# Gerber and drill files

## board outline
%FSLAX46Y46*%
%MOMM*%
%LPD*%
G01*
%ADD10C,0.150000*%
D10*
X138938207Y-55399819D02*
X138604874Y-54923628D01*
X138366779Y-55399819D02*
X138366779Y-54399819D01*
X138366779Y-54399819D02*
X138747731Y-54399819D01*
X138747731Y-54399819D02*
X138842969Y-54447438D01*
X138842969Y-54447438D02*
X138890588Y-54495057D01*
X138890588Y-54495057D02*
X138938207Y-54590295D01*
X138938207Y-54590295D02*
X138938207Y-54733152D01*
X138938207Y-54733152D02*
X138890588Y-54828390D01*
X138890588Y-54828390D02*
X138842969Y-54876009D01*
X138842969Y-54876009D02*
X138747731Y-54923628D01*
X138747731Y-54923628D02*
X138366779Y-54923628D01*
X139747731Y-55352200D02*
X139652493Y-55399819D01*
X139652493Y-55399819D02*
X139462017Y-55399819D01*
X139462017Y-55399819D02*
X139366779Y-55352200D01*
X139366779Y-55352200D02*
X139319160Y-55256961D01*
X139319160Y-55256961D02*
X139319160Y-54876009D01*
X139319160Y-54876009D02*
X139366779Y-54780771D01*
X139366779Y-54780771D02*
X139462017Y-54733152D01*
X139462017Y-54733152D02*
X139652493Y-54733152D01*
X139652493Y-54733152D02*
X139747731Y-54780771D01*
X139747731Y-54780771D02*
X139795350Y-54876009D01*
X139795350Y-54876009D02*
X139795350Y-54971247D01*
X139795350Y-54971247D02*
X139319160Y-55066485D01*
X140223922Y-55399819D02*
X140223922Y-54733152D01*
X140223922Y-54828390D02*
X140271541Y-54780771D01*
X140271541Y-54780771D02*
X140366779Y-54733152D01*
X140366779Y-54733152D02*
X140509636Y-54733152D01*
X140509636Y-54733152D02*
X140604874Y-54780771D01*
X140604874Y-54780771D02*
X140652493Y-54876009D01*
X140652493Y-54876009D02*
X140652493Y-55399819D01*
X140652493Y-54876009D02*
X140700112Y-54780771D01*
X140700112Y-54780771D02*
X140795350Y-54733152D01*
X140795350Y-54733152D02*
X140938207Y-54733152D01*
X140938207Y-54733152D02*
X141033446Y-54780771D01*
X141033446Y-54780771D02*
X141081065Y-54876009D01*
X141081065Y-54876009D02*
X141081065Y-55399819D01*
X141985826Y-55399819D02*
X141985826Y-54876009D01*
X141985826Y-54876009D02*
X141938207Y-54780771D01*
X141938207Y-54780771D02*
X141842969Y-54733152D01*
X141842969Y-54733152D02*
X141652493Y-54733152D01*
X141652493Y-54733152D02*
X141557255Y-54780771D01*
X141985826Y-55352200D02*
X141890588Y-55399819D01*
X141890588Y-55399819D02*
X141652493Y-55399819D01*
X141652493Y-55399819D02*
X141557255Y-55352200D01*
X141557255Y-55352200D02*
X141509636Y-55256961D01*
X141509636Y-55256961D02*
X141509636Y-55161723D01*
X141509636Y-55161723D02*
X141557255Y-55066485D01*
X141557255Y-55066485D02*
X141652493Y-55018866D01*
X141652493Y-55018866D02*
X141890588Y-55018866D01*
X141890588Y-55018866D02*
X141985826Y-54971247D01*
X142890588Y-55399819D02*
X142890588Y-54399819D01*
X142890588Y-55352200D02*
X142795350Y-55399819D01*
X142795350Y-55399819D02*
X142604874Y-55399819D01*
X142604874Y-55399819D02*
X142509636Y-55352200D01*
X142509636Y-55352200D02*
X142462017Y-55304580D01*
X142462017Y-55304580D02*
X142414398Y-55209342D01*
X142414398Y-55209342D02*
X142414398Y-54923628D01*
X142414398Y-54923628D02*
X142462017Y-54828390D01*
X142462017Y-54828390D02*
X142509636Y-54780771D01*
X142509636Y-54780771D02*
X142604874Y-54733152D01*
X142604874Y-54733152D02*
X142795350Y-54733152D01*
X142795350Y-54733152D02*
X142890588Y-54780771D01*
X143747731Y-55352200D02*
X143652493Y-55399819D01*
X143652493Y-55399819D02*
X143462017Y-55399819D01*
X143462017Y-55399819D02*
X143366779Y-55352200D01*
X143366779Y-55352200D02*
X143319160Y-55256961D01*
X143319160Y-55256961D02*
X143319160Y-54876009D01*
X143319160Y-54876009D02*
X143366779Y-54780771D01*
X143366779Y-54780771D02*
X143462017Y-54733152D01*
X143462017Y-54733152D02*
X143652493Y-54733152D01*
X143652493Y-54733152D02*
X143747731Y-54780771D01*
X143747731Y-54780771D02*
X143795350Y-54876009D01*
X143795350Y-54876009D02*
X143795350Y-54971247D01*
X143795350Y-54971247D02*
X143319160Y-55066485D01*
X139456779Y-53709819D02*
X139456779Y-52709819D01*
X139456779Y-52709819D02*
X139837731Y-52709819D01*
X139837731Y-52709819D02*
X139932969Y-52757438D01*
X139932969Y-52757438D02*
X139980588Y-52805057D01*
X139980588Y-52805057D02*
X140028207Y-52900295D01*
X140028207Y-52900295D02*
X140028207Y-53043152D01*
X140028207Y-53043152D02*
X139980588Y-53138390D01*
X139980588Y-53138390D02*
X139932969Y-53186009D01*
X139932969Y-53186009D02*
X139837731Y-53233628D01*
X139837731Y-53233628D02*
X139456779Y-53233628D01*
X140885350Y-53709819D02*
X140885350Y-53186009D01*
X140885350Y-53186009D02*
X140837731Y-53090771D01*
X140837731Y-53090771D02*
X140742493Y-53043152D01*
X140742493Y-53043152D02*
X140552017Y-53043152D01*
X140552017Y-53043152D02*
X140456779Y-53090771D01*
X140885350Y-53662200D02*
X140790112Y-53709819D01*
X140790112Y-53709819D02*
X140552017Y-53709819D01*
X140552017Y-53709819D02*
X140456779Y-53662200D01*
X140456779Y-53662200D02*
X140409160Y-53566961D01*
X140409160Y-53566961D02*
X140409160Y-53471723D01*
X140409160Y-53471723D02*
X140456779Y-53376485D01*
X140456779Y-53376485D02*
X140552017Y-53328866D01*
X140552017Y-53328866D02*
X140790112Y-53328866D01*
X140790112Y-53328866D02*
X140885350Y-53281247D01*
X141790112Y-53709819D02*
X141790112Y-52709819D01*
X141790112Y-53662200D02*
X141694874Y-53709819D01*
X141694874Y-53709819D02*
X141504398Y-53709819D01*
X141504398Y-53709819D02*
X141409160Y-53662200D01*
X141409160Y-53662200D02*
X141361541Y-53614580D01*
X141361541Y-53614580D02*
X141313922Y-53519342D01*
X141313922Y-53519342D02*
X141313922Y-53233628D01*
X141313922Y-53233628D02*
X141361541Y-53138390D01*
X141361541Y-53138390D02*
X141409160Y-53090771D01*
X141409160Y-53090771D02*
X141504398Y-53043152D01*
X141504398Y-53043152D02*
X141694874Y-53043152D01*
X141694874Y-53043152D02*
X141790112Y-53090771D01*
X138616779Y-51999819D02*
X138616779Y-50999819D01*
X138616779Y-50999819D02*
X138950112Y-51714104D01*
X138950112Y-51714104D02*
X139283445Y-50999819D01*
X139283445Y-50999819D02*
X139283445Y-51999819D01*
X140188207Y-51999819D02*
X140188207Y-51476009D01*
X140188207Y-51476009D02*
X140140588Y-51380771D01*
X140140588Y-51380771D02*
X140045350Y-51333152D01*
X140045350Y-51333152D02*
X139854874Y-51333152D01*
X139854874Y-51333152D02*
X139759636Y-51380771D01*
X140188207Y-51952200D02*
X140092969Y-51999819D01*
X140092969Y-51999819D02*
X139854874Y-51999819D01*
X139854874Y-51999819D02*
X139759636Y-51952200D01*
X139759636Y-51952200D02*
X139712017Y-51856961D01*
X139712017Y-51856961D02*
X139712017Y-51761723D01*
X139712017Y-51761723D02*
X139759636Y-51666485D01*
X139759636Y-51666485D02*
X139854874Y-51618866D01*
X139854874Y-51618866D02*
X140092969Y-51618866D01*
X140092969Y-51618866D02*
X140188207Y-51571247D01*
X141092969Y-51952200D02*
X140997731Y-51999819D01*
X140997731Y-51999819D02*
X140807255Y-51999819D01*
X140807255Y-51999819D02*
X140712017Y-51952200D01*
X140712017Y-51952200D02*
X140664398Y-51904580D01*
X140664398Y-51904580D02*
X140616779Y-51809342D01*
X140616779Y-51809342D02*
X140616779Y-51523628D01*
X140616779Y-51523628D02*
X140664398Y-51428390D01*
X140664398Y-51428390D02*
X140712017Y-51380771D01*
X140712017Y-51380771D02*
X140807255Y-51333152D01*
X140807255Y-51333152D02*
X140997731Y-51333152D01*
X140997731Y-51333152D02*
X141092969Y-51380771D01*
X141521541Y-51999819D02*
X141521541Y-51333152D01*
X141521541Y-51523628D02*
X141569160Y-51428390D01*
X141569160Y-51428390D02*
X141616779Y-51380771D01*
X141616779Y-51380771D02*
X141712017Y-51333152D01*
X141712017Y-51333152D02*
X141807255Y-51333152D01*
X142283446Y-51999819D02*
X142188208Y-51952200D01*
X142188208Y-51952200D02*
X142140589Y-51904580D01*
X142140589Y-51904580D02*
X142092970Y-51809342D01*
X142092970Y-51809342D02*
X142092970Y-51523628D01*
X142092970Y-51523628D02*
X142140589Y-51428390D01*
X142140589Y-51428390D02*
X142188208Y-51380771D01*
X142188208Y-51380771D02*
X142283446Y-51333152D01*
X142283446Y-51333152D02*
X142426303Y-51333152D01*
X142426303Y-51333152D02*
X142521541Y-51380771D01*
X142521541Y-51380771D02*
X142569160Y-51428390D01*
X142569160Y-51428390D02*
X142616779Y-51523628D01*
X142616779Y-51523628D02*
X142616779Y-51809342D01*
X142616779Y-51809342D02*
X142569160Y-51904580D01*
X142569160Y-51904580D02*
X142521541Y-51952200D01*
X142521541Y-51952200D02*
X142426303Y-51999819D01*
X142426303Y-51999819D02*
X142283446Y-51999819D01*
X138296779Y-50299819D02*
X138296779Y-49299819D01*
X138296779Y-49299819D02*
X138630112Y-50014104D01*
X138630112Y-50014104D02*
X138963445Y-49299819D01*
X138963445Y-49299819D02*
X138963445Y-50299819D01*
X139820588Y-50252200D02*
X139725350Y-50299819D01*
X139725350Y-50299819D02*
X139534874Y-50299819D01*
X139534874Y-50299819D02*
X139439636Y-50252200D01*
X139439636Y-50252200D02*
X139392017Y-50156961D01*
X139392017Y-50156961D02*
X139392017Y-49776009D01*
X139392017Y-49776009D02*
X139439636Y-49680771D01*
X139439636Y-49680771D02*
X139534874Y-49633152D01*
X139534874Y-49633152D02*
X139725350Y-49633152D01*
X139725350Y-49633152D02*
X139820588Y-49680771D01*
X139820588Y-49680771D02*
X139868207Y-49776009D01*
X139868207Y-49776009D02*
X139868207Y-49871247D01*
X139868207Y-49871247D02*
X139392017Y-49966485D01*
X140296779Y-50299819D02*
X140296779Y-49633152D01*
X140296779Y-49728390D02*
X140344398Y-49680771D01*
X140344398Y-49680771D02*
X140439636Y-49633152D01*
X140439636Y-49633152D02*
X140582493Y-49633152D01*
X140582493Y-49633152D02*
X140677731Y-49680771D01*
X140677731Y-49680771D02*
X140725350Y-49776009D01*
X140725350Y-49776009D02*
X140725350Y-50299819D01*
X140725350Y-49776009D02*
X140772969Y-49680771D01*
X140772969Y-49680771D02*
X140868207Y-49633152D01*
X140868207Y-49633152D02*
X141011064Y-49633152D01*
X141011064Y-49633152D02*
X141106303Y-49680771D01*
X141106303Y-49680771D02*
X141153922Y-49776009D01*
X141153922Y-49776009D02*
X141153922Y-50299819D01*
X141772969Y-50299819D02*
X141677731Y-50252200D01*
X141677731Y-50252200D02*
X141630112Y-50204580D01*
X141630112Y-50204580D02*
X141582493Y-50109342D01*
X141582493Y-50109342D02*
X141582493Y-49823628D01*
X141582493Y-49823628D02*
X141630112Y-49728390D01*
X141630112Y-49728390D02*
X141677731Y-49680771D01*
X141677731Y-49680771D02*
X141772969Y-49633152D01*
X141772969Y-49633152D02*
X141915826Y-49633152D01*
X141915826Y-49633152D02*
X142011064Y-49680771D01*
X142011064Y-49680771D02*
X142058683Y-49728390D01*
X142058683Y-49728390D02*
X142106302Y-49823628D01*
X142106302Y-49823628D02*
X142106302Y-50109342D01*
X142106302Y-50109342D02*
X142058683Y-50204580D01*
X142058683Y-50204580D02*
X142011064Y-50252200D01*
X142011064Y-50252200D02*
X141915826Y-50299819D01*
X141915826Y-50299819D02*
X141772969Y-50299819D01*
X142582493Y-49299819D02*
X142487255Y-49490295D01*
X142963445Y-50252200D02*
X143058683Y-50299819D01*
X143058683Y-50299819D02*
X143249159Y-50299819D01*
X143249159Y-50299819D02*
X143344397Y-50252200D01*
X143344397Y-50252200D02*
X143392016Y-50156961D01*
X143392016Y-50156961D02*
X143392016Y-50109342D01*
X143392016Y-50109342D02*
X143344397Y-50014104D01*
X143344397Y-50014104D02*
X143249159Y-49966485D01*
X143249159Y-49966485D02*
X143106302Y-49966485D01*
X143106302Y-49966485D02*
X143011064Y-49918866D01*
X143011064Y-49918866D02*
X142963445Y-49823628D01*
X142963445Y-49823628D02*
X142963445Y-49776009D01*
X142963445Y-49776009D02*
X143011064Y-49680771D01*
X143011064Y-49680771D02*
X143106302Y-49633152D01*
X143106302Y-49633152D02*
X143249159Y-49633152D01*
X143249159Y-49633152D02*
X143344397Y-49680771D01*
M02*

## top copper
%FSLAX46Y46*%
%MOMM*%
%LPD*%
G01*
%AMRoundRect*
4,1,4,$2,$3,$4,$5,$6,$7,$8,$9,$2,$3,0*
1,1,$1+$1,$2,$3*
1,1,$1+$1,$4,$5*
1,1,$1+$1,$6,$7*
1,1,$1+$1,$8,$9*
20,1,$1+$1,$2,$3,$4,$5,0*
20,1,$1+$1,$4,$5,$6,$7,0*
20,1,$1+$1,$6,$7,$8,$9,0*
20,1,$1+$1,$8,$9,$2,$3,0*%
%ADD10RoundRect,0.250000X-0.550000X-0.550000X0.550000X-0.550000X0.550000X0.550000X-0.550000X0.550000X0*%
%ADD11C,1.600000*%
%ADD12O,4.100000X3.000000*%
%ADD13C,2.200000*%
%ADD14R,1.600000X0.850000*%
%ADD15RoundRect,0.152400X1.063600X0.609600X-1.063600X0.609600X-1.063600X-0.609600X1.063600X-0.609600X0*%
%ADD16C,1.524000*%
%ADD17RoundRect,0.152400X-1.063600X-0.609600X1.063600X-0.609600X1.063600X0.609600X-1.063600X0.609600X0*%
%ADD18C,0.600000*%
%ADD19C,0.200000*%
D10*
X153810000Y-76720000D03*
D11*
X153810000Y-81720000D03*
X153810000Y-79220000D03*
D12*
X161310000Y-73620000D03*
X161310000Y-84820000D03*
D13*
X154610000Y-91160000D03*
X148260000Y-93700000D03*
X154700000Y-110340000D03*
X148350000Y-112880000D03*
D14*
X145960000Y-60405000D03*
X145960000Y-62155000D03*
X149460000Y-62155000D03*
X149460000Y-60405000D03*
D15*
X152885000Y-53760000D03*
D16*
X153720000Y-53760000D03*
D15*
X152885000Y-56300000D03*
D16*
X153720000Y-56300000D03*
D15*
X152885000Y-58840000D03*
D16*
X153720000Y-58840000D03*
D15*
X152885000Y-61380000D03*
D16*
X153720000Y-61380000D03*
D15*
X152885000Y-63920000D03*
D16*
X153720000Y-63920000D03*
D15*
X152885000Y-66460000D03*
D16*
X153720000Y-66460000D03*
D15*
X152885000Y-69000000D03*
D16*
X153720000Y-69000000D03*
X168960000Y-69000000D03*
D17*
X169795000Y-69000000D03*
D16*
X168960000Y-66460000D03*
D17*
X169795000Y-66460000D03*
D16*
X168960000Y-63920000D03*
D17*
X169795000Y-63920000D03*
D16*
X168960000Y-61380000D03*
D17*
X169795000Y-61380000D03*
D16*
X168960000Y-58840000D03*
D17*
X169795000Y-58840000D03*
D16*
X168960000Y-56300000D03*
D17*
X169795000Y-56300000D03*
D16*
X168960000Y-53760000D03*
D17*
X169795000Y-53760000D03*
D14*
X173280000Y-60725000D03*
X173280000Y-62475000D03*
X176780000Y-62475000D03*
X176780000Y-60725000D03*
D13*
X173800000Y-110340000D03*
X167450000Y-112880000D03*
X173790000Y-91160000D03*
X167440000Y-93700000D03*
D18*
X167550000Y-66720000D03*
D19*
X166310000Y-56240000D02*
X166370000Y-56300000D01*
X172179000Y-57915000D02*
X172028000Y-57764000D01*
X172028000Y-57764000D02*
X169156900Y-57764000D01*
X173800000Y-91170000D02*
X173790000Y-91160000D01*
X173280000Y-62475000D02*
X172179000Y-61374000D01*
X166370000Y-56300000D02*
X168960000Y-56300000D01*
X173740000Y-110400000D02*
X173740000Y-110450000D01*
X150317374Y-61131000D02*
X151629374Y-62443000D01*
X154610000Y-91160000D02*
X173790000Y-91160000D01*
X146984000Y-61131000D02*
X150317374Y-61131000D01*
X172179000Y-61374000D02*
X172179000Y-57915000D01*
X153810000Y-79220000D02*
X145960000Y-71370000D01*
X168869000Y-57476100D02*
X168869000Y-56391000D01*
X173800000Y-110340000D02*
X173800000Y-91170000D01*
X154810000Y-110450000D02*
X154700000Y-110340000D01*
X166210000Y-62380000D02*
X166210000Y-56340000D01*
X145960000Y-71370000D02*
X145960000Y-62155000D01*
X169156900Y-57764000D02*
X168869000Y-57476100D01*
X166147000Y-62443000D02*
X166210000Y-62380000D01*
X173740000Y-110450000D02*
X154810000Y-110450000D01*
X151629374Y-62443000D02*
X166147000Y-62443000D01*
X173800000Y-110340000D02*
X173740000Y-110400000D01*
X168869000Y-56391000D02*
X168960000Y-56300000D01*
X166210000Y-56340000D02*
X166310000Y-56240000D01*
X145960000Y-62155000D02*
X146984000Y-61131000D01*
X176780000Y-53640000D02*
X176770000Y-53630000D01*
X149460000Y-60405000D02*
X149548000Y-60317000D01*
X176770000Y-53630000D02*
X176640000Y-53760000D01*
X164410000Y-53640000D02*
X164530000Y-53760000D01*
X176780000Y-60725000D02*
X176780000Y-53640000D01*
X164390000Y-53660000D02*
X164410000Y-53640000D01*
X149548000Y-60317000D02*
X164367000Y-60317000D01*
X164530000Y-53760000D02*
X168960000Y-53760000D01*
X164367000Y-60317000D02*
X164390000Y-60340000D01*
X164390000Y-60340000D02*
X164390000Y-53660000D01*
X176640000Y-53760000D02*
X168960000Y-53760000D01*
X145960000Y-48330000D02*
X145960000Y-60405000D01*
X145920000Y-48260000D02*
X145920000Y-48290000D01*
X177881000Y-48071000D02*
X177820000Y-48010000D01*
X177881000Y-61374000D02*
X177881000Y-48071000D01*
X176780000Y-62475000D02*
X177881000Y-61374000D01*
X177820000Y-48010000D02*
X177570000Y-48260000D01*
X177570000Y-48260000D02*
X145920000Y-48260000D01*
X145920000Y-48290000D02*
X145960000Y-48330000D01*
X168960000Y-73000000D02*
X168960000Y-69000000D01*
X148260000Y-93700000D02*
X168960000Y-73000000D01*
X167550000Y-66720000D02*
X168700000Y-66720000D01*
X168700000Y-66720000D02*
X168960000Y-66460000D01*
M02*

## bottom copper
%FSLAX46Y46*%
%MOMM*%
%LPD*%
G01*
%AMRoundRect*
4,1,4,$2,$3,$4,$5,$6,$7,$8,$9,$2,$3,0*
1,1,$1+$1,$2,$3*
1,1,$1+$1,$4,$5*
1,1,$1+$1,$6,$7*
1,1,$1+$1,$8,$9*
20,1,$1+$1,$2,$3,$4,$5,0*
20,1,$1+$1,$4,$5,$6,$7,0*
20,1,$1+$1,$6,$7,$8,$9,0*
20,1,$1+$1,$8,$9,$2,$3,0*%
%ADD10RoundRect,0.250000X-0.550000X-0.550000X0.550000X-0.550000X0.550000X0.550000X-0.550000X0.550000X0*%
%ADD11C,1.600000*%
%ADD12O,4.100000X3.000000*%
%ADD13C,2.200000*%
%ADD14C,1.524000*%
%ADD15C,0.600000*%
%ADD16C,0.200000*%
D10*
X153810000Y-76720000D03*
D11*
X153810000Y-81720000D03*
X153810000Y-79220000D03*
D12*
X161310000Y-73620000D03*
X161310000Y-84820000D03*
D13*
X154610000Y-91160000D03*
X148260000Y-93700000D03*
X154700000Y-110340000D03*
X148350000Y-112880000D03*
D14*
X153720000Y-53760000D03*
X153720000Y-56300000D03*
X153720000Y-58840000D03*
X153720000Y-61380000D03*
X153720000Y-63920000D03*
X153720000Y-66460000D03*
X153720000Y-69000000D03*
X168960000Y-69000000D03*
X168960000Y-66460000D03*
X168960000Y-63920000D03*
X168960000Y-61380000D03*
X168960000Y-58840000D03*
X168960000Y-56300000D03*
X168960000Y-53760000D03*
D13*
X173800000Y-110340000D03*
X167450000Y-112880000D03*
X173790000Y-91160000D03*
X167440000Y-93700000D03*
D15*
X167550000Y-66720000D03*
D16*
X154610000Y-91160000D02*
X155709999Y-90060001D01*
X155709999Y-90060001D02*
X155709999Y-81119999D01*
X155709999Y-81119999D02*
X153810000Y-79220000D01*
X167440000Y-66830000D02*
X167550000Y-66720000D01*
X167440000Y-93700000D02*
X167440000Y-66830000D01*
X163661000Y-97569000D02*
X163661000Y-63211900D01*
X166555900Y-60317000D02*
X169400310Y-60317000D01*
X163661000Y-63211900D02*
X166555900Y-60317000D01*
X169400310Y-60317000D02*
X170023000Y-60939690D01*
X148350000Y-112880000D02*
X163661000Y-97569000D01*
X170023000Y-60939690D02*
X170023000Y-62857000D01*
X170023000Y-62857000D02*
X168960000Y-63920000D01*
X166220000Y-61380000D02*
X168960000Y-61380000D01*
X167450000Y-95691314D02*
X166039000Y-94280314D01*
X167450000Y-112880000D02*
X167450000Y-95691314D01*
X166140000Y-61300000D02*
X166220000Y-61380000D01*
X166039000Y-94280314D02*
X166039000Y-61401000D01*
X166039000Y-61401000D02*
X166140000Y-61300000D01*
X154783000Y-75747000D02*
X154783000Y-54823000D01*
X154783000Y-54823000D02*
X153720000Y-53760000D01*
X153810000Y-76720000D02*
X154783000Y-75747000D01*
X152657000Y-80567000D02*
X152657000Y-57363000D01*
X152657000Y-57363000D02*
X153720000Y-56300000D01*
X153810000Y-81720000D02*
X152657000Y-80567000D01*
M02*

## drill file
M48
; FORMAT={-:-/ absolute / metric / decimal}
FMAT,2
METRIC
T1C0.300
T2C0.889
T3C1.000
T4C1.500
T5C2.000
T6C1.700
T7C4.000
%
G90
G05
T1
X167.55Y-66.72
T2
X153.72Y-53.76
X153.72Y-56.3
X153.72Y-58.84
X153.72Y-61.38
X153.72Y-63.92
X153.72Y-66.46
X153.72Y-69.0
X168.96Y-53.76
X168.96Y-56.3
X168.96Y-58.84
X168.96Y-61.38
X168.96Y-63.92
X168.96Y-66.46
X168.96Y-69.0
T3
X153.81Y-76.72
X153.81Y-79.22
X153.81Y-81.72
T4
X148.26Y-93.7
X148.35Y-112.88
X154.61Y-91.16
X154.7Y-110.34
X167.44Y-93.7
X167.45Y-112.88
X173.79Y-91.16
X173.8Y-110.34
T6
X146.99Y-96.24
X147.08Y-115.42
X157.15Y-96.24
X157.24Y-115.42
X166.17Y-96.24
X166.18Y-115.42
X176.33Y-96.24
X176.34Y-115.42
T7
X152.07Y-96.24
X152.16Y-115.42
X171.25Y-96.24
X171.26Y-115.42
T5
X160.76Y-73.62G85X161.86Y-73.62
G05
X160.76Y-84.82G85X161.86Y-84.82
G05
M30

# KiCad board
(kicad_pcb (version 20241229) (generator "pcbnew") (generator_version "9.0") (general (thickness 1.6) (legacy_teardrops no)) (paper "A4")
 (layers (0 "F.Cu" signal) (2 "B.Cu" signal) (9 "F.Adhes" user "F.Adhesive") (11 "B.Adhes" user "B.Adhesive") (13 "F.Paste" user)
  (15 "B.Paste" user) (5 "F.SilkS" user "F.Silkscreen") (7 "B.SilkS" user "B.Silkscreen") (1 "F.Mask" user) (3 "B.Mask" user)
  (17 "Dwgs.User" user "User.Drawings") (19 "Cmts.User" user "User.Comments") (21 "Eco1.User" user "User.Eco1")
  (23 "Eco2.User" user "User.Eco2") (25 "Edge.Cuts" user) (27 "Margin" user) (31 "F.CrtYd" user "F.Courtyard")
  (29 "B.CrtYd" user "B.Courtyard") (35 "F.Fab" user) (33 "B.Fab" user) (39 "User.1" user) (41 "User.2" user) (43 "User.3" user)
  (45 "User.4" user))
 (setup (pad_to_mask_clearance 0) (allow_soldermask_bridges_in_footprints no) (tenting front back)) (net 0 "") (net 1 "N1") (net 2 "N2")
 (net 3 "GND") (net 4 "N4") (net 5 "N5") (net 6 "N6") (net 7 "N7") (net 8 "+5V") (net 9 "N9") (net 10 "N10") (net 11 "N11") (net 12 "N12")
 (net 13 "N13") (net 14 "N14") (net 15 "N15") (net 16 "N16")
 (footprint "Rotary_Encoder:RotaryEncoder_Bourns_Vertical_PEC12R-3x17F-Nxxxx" (layer "F.Cu") (at 153.81 76.72)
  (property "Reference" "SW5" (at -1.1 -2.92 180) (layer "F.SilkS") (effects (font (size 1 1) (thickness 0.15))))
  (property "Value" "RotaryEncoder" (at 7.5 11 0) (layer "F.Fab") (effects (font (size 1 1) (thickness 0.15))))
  (pad "A" thru_hole roundrect (at 0 0) (size 1.6 1.6) (drill 1) (layers "*.Cu" "*.Mask") (remove_unused_layers no)
   (roundrect_rratio 0.15625) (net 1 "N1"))
  (pad "B" thru_hole circle (at 0 5) (size 1.6 1.6) (drill 1) (layers "*.Cu" "*.Mask") (remove_unused_layers no) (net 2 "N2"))
  (pad "C" thru_hole circle (at 0 2.5) (size 1.6 1.6) (drill 1) (layers "*.Cu" "*.Mask") (remove_unused_layers no) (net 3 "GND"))
  (pad "SH" thru_hole oval (at 7.5 -3.1) (size 4.1 3) (drill oval 3.1 2) (layers "*.Cu" "*.Mask") (remove_unused_layers no))
  (pad "SH" thru_hole oval (at 7.5 8.1) (size 4.1 3) (drill oval 3.1 2) (layers "*.Cu" "*.Mask") (remove_unused_layers no)))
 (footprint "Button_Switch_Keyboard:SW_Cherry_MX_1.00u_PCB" (layer "F.Cu") (at 154.61 91.16)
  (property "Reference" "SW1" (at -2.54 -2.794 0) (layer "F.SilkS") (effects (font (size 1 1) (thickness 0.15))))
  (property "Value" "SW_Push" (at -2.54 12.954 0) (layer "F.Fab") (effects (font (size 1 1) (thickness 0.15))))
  (pad "" np_thru_hole circle (at -7.62 5.08) (size 1.7 1.7) (drill 1.7) (layers "*.Cu" "*.Mask"))
  (pad "" np_thru_hole circle (at -2.54 5.08) (size 4 4) (drill 4) (layers "*.Cu" "*.Mask"))
  (pad "" np_thru_hole circle (at 2.54 5.08) (size 1.7 1.7) (drill 1.7) (layers "*.Cu" "*.Mask"))
  (pad "1" thru_hole circle (at 0 0) (size 2.2 2.2) (drill 1.5) (layers "*.Cu" "*.Mask") (remove_unused_layers no) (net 3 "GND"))
  (pad "2" thru_hole circle (at -6.35 2.54) (size 2.2 2.2) (drill 1.5) (layers "*.Cu" "*.Mask") (remove_unused_layers no) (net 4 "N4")))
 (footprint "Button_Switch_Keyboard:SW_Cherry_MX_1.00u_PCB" (layer "F.Cu") (at 154.7 110.34)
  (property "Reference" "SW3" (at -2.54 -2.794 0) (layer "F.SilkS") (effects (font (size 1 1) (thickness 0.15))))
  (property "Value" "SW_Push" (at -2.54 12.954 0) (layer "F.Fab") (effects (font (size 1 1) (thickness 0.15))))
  (pad "" np_thru_hole circle (at -7.62 5.08) (size 1.7 1.7) (drill 1.7) (layers "*.Cu" "*.Mask"))
  (pad "" np_thru_hole circle (at -2.54 5.08) (size 4 4) (drill 4) (layers "*.Cu" "*.Mask"))
  (pad "" np_thru_hole circle (at 2.54 5.08) (size 1.7 1.7) (drill 1.7) (layers "*.Cu" "*.Mask"))
  (pad "1" thru_hole circle (at 0 0) (size 2.2 2.2) (drill 1.5) (layers "*.Cu" "*.Mask") (remove_unused_layers no) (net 3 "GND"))
  (pad "2" thru_hole circle (at -6.35 2.54) (size 2.2 2.2) (drill 1.5) (layers "*.Cu" "*.Mask") (remove_unused_layers no) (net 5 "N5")))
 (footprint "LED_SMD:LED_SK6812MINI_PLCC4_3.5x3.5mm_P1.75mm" (layer "F.Cu") (at 147.71 61.28)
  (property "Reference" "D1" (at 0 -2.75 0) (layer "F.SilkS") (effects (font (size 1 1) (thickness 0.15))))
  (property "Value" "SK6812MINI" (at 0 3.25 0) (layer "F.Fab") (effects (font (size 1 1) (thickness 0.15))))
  (pad "1" smd rect (at -1.75 -0.875) (size 1.6 0.85) (layers "F.Cu" "F.Mask" "F.Paste") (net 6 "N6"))
  (pad "2" smd rect (at -1.75 0.875) (size 1.6 0.85) (layers "F.Cu" "F.Mask" "F.Paste") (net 3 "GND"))
  (pad "3" smd rect (at 1.75 0.875) (size 1.6 0.85) (layers "F.Cu" "F.Mask" "F.Paste") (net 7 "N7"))
  (pad "4" smd rect (at 1.75 -0.875) (size 1.6 0.85) (layers "F.Cu" "F.Mask" "F.Paste") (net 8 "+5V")))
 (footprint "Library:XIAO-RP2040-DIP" (layer "F.Cu") (at 161.34 61.38)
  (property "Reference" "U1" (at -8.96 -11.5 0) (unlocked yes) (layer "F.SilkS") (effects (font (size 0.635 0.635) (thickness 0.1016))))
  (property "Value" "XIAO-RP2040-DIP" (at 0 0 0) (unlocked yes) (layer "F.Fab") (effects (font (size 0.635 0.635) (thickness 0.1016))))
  (pad "1" smd roundrect (at -8.455 -7.62 180) (size 2.432 1.524) (layers "F.Cu" "F.Mask") (roundrect_rratio 0.1) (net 1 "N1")
   (thermal_bridge_angle 45))
  (pad "1" thru_hole circle (at -7.62 -7.62 180) (size 1.524 1.524) (drill 0.889) (layers "*.Cu" "*.Mask") (remove_unused_layers no)
   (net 1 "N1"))
  (pad "2" smd roundrect (at -8.455 -5.08 180) (size 2.432 1.524) (layers "F.Cu" "F.Mask") (roundrect_rratio 0.1) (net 2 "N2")
   (thermal_bridge_angle 45))
  (pad "2" thru_hole circle (at -7.62 -5.08 180) (size 1.524 1.524) (drill 0.889) (layers "*.Cu" "*.Mask") (remove_unused_layers no)
   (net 2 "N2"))
  (pad "3" smd roundrect (at -8.455 -2.54 180) (size 2.432 1.524) (layers "F.Cu" "F.Mask") (roundrect_rratio 0.1) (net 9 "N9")
   (thermal_bridge_angle 45))
  (pad "3" thru_hole circle (at -7.62 -2.54 180) (size 1.524 1.524) (drill 0.889) (layers "*.Cu" "*.Mask") (remove_unused_layers no)
   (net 9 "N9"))
  (pad "4" smd roundrect (at -8.455 0 180) (size 2.432 1.524) (layers "F.Cu" "F.Mask") (roundrect_rratio 0.1) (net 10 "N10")
   (thermal_bridge_angle 45))
  (pad "4" thru_hole circle (at -7.62 0 180) (size 1.524 1.524) (drill 0.889) (layers "*.Cu" "*.Mask") (remove_unused_layers no)
   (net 10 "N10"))
  (pad "5" smd roundrect (at -8.455 2.54 180) (size 2.432 1.524) (layers "F.Cu" "F.Mask") (roundrect_rratio 0.1) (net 7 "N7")
   (thermal_bridge_angle 45))
  (pad "5" thru_hole circle (at -7.62 2.54 180) (size 1.524 1.524) (drill 0.889) (layers "*.Cu" "*.Mask") (remove_unused_layers no)
   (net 7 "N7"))
  (pad "6" smd roundrect (at -8.455 5.08 180) (size 2.432 1.524) (layers "F.Cu" "F.Mask") (roundrect_rratio 0.1) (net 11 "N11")
   (thermal_bridge_angle 45))
  (pad "6" thru_hole circle (at -7.62 5.08 180) (size 1.524 1.524) (drill 0.889) (layers "*.Cu" "*.Mask") (remove_unused_layers no)
   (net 11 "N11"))
  (pad "7" smd roundrect (at -8.455 7.62 180) (size 2.432 1.524) (layers "F.Cu" "F.Mask") (roundrect_rratio 0.1) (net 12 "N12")
   (thermal_bridge_angle 45))
  (pad "7" thru_hole circle (at -7.62 7.62 180) (size 1.524 1.524) (drill 0.889) (layers "*.Cu" "*.Mask") (remove_unused_layers no)
   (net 12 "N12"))
  (pad "8" thru_hole circle (at 7.62 7.62) (size 1.524 1.524) (drill 0.889) (layers "*.Cu" "*.Mask") (remove_unused_layers no) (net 4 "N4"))
  (pad "8" smd roundrect (at 8.455 7.62) (size 2.432 1.524) (layers "F.Cu" "F.Mask") (roundrect_rratio 0.1) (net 4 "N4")
   (thermal_bridge_angle 45))
  (pad "9" thru_hole circle (at 7.62 5.08) (size 1.524 1.524) (drill 0.889) (layers "*.Cu" "*.Mask") (remove_unused_layers no)
   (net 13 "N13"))
  (pad "9" smd roundrect (at 8.455 5.08) (size 2.432 1.524) (layers "F.Cu" "F.Mask") (roundrect_rratio 0.1) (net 13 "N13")
   (thermal_bridge_angle 45))
  (pad "10" thru_hole circle (at 7.62 2.54) (size 1.524 1.524) (drill 0.889) (layers "*.Cu" "*.Mask") (remove_unused_layers no) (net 5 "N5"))
  (pad "10" smd roundrect (at 8.455 2.54) (size 2.432 1.524) (layers "F.Cu" "F.Mask") (roundrect_rratio 0.1) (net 5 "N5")
   (thermal_bridge_angle 45))
  (pad "11" thru_hole circle (at 7.62 0) (size 1.524 1.524) (drill 0.889) (layers "*.Cu" "*.Mask") (remove_unused_layers no) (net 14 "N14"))
  (pad "11" smd roundrect (at 8.455 0) (size 2.432 1.524) (layers "F.Cu" "F.Mask") (roundrect_rratio 0.1) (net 14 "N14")
   (thermal_bridge_angle 45))
  (pad "12" thru_hole circle (at 7.62 -2.54) (size 1.524 1.524) (drill 0.889) (layers "*.Cu" "*.Mask") (remove_unused_layers no)
   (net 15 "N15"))
  (pad "12" smd roundrect (at 8.455 -2.54) (size 2.432 1.524) (layers "F.Cu" "F.Mask") (roundrect_rratio 0.1) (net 15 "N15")
   (thermal_bridge_angle 45))
  (pad "13" thru_hole circle (at 7.62 -5.08) (size 1.524 1.524) (drill 0.889) (layers "*.Cu" "*.Mask") (remove_unused_layers no)
   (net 3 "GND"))
  (pad "13" smd roundrect (at 8.455 -5.08) (size 2.432 1.524) (layers "F.Cu" "F.Mask") (roundrect_rratio 0.1) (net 3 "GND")
   (thermal_bridge_angle 45))
  (pad "14" thru_hole circle (at 7.62 -7.62) (size 1.524 1.524) (drill 0.889) (layers "*.Cu" "*.Mask") (remove_unused_layers no)
   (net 8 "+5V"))
  (pad "14" smd roundrect (at 8.455 -7.62) (size 2.432 1.524) (layers "F.Cu" "F.Mask") (roundrect_rratio 0.1) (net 8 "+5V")
   (thermal_bridge_angle 45)))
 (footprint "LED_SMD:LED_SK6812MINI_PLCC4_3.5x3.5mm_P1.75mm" (layer "F.Cu") (at 175.03 61.6)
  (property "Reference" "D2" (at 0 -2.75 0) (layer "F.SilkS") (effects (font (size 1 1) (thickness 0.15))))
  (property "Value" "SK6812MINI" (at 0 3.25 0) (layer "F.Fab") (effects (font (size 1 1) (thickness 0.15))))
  (pad "1" smd rect (at -1.75 -0.875) (size 1.6 0.85) (layers "F.Cu" "F.Mask" "F.Paste") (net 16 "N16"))
  (pad "2" smd rect (at -1.75 0.875) (size 1.6 0.85) (layers "F.Cu" "F.Mask" "F.Paste") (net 3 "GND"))
  (pad "3" smd rect (at 1.75 0.875) (size 1.6 0.85) (layers "F.Cu" "F.Mask" "F.Paste") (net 6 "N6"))
  (pad "4" smd rect (at 1.75 -0.875) (size 1.6 0.85) (layers "F.Cu" "F.Mask" "F.Paste") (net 8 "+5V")))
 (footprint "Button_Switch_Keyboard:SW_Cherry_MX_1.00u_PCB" (layer "F.Cu") (at 173.8 110.34)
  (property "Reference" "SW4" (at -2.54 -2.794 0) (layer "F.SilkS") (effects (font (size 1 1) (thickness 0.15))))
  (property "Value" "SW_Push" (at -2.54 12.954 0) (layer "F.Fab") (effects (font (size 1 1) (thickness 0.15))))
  (pad "" np_thru_hole circle (at -7.62 5.08) (size 1.7 1.7) (drill 1.7) (layers "*.Cu" "*.Mask"))
  (pad "" np_thru_hole circle (at -2.54 5.08) (size 4 4) (drill 4) (layers "*.Cu" "*.Mask"))
  (pad "" np_thru_hole circle (at 2.54 5.08) (size 1.7 1.7) (drill 1.7) (layers "*.Cu" "*.Mask"))
  (pad "1" thru_hole circle (at 0 0) (size 2.2 2.2) (drill 1.5) (layers "*.Cu" "*.Mask") (remove_unused_layers no) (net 3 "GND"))
  (pad "2" thru_hole circle (at -6.35 2.54) (size 2.2 2.2) (drill 1.5) (layers "*.Cu" "*.Mask") (remove_unused_layers no) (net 14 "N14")))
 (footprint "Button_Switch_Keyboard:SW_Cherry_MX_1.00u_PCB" (layer "F.Cu") (at 173.79 91.16)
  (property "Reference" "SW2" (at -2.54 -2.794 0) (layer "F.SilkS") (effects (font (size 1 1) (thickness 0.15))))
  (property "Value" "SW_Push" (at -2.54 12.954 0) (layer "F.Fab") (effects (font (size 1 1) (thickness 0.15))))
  (pad "" np_thru_hole circle (at -7.62 5.08) (size 1.7 1.7) (drill 1.7) (layers "*.Cu" "*.Mask"))
  (pad "" np_thru_hole circle (at -2.54 5.08) (size 4 4) (drill 4) (layers "*.Cu" "*.Mask"))
  (pad "" np_thru_hole circle (at 2.54 5.08) (size 1.7 1.7) (drill 1.7) (layers "*.Cu" "*.Mask"))
  (pad "1" thru_hole circle (at 0 0) (size 2.2 2.2) (drill 1.5) (layers "*.Cu" "*.Mask") (remove_unused_layers no) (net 3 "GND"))
  (pad "2" thru_hole circle (at -6.35 2.54) (size 2.2 2.2) (drill 1.5) (layers "*.Cu" "*.Mask") (remove_unused_layers no) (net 13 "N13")))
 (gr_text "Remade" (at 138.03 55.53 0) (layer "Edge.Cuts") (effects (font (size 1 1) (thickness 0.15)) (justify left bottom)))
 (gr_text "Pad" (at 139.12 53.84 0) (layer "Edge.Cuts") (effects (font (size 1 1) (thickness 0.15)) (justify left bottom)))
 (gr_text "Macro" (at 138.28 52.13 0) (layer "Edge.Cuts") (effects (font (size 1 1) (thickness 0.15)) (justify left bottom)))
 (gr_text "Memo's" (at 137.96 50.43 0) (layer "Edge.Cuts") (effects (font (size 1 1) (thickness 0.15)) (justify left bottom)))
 (segment (start 166.31 56.24) (end 166.37 56.3) (width 0.2) (layer "F.Cu") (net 3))
 (segment (start 172.179 57.915) (end 172.028 57.764) (width 0.2) (layer "F.Cu") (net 3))
 (segment (start 172.028 57.764) (end 169.1569 57.764) (width 0.2) (layer "F.Cu") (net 3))
 (segment (start 173.8 91.17) (end 173.79 91.16) (width 0.2) (layer "F.Cu") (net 3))
 (segment (start 173.28 62.475) (end 172.179 61.374) (width 0.2) (layer "F.Cu") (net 3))
 (segment (start 166.37 56.3) (end 168.96 56.3) (width 0.2) (layer "F.Cu") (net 3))
 (segment (start 173.74 110.4) (end 173.74 110.45) (width 0.2) (layer "F.Cu") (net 3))
 (segment (start 150.317374 61.131) (end 151.629374 62.443) (width 0.2) (layer "F.Cu") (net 3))
 (segment (start 154.61 91.16) (end 173.79 91.16) (width 0.2) (layer "F.Cu") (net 3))
 (segment (start 146.984 61.131) (end 150.317374 61.131) (width 0.2) (layer "F.Cu") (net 3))
 (segment (start 172.179 61.374) (end 172.179 57.915) (width 0.2) (layer "F.Cu") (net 3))
 (segment (start 153.81 79.22) (end 145.96 71.37) (width 0.2) (layer "F.Cu") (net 3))
 (segment (start 168.869 57.4761) (end 168.869 56.391) (width 0.2) (layer "F.Cu") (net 3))
 (segment (start 173.8 110.34) (end 173.8 91.17) (width 0.2) (layer "F.Cu") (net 3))
 (segment (start 154.81 110.45) (end 154.7 110.34) (width 0.2) (layer "F.Cu") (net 3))
 (segment (start 166.21 62.38) (end 166.21 56.34) (width 0.2) (layer "F.Cu") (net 3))
 (segment (start 145.96 71.37) (end 145.96 62.155) (width 0.2) (layer "F.Cu") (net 3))
 (segment (start 169.1569 57.764) (end 168.869 57.4761) (width 0.2) (layer "F.Cu") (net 3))
 (segment (start 166.147 62.443) (end 166.21 62.38) (width 0.2) (layer "F.Cu") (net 3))
 (segment (start 173.74 110.45) (end 154.81 110.45) (width 0.2) (layer "F.Cu") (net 3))
 (segment (start 151.629374 62.443) (end 166.147 62.443) (width 0.2) (layer "F.Cu") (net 3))
 (segment (start 173.8 110.34) (end 173.74 110.4) (width 0.2) (layer "F.Cu") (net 3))
 (segment (start 168.869 56.391) (end 168.96 56.3) (width 0.2) (layer "F.Cu") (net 3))
 (segment (start 166.21 56.34) (end 166.31 56.24) (width 0.2) (layer "F.Cu") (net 3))
 (segment (start 145.96 62.155) (end 146.984 61.131) (width 0.2) (layer "F.Cu") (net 3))
 (segment (start 154.61 91.16) (end 155.709999 90.060001) (width 0.2) (layer "B.Cu") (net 3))
 (segment (start 155.709999 90.060001) (end 155.709999 81.119999) (width 0.2) (layer "B.Cu") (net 3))
 (segment (start 155.709999 81.119999) (end 153.81 79.22) (width 0.2) (layer "B.Cu") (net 3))
 (segment (start 176.78 53.64) (end 176.77 53.63) (width 0.2) (layer "F.Cu") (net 8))
 (segment (start 149.46 60.405) (end 149.548 60.317) (width 0.2) (layer "F.Cu") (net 8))
 (segment (start 176.77 53.63) (end 176.64 53.76) (width 0.2) (layer "F.Cu") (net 8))
 (segment (start 164.41 53.64) (end 164.53 53.76) (width 0.2) (layer "F.Cu") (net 8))
 (segment (start 176.78 60.725) (end 176.78 53.64) (width 0.2) (layer "F.Cu") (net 8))
 (segment (start 164.39 53.66) (end 164.41 53.64) (width 0.2) (layer "F.Cu") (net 8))
 (segment (start 149.548 60.317) (end 164.367 60.317) (width 0.2) (layer "F.Cu") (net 8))
 (segment (start 164.53 53.76) (end 168.96 53.76) (width 0.2) (layer "F.Cu") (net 8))
 (segment (start 164.367 60.317) (end 164.39 60.34) (width 0.2) (layer "F.Cu") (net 8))
 (segment (start 164.39 60.34) (end 164.39 53.66) (width 0.2) (layer "F.Cu") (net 8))
 (segment (start 176.64 53.76) (end 168.96 53.76) (width 0.2) (layer "F.Cu") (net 8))
 (segment (start 145.96 48.33) (end 145.96 60.405) (width 0.2) (layer "F.Cu") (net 6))
 (segment (start 145.92 48.26) (end 145.92 48.29) (width 0.2) (layer "F.Cu") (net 6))
 (segment (start 177.881 48.071) (end 177.82 48.01) (width 0.2) (layer "F.Cu") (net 6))
 (segment (start 177.881 61.374) (end 177.881 48.071) (width 0.2) (layer "F.Cu") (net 6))
 (segment (start 176.78 62.475) (end 177.881 61.374) (width 0.2) (layer "F.Cu") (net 6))
 (segment (start 177.82 48.01) (end 177.57 48.26) (width 0.2) (layer "F.Cu") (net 6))
 (segment (start 177.57 48.26) (end 145.92 48.26) (width 0.2) (layer "F.Cu") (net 6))
 (segment (start 145.92 48.29) (end 145.96 48.33) (width 0.2) (layer "F.Cu") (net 6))
 (segment (start 168.96 73) (end 168.96 69) (width 0.2) (layer "F.Cu") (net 4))
 (segment (start 148.26 93.7) (end 168.96 73) (width 0.2) (layer "F.Cu") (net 4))
 (segment (start 167.55 66.72) (end 168.7 66.72) (width 0.2) (layer "F.Cu") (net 13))
 (segment (start 168.7 66.72) (end 168.96 66.46) (width 0.2) (layer "F.Cu") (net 13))
 (via (at 167.55 66.72) (size 0.6) (drill 0.3) (layers "F.Cu" "B.Cu") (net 13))
 (segment (start 167.44 66.83) (end 167.55 66.72) (width 0.2) (layer "B.Cu") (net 13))
 (segment (start 167.44 93.7) (end 167.44 66.83) (width 0.2) (layer "B.Cu") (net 13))
 (segment (start 163.661 97.569) (end 163.661 63.2119) (width 0.2) (layer "B.Cu") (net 5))
 (segment (start 166.5559 60.317) (end 169.40031 60.317) (width 0.2) (layer "B.Cu") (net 5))
 (segment (start 163.661 63.2119) (end 166.5559 60.317) (width 0.2) (layer "B.Cu") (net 5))
 (segment (start 169.40031 60.317) (end 170.023 60.93969) (width 0.2) (layer "B.Cu") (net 5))
 (segment (start 148.35 112.88) (end 163.661 97.569) (width 0.2) (layer "B.Cu") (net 5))
 (segment (start 170.023 60.93969) (end 170.023 62.857) (width 0.2) (layer "B.Cu") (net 5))
 (segment (start 170.023 62.857) (end 168.96 63.92) (width 0.2) (layer "B.Cu") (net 5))
 (segment (start 166.22 61.38) (end 168.96 61.38) (width 0.2) (layer "B.Cu") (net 14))
 (segment (start 167.45 95.691314) (end 166.039 94.280314) (width 0.2) (layer "B.Cu") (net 14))
 (segment (start 167.45 112.88) (end 167.45 95.691314) (width 0.2) (layer "B.Cu") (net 14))
 (segment (start 166.14 61.3) (end 166.22 61.38) (width 0.2) (layer "B.Cu") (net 14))
 (segment (start 166.039 94.280314) (end 166.039 61.401) (width 0.2) (layer "B.Cu") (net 14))
 (segment (start 166.039 61.401) (end 166.14 61.3) (width 0.2) (layer "B.Cu") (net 14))
 (segment (start 154.783 75.747) (end 154.783 54.823) (width 0.2) (layer "B.Cu") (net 1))
 (segment (start 154.783 54.823) (end 153.72 53.76) (width 0.2) (layer "B.Cu") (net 1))
 (segment (start 153.81 76.72) (end 154.783 75.747) (width 0.2) (layer "B.Cu") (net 1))
 (segment (start 152.657 80.567) (end 152.657 57.363) (width 0.2) (layer "B.Cu") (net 2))
 (segment (start 152.657 57.363) (end 153.72 56.3) (width 0.2) (layer "B.Cu") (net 2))
 (segment (start 153.81 81.72) (end 152.657 80.567) (width 0.2) (layer "B.Cu") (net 2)))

